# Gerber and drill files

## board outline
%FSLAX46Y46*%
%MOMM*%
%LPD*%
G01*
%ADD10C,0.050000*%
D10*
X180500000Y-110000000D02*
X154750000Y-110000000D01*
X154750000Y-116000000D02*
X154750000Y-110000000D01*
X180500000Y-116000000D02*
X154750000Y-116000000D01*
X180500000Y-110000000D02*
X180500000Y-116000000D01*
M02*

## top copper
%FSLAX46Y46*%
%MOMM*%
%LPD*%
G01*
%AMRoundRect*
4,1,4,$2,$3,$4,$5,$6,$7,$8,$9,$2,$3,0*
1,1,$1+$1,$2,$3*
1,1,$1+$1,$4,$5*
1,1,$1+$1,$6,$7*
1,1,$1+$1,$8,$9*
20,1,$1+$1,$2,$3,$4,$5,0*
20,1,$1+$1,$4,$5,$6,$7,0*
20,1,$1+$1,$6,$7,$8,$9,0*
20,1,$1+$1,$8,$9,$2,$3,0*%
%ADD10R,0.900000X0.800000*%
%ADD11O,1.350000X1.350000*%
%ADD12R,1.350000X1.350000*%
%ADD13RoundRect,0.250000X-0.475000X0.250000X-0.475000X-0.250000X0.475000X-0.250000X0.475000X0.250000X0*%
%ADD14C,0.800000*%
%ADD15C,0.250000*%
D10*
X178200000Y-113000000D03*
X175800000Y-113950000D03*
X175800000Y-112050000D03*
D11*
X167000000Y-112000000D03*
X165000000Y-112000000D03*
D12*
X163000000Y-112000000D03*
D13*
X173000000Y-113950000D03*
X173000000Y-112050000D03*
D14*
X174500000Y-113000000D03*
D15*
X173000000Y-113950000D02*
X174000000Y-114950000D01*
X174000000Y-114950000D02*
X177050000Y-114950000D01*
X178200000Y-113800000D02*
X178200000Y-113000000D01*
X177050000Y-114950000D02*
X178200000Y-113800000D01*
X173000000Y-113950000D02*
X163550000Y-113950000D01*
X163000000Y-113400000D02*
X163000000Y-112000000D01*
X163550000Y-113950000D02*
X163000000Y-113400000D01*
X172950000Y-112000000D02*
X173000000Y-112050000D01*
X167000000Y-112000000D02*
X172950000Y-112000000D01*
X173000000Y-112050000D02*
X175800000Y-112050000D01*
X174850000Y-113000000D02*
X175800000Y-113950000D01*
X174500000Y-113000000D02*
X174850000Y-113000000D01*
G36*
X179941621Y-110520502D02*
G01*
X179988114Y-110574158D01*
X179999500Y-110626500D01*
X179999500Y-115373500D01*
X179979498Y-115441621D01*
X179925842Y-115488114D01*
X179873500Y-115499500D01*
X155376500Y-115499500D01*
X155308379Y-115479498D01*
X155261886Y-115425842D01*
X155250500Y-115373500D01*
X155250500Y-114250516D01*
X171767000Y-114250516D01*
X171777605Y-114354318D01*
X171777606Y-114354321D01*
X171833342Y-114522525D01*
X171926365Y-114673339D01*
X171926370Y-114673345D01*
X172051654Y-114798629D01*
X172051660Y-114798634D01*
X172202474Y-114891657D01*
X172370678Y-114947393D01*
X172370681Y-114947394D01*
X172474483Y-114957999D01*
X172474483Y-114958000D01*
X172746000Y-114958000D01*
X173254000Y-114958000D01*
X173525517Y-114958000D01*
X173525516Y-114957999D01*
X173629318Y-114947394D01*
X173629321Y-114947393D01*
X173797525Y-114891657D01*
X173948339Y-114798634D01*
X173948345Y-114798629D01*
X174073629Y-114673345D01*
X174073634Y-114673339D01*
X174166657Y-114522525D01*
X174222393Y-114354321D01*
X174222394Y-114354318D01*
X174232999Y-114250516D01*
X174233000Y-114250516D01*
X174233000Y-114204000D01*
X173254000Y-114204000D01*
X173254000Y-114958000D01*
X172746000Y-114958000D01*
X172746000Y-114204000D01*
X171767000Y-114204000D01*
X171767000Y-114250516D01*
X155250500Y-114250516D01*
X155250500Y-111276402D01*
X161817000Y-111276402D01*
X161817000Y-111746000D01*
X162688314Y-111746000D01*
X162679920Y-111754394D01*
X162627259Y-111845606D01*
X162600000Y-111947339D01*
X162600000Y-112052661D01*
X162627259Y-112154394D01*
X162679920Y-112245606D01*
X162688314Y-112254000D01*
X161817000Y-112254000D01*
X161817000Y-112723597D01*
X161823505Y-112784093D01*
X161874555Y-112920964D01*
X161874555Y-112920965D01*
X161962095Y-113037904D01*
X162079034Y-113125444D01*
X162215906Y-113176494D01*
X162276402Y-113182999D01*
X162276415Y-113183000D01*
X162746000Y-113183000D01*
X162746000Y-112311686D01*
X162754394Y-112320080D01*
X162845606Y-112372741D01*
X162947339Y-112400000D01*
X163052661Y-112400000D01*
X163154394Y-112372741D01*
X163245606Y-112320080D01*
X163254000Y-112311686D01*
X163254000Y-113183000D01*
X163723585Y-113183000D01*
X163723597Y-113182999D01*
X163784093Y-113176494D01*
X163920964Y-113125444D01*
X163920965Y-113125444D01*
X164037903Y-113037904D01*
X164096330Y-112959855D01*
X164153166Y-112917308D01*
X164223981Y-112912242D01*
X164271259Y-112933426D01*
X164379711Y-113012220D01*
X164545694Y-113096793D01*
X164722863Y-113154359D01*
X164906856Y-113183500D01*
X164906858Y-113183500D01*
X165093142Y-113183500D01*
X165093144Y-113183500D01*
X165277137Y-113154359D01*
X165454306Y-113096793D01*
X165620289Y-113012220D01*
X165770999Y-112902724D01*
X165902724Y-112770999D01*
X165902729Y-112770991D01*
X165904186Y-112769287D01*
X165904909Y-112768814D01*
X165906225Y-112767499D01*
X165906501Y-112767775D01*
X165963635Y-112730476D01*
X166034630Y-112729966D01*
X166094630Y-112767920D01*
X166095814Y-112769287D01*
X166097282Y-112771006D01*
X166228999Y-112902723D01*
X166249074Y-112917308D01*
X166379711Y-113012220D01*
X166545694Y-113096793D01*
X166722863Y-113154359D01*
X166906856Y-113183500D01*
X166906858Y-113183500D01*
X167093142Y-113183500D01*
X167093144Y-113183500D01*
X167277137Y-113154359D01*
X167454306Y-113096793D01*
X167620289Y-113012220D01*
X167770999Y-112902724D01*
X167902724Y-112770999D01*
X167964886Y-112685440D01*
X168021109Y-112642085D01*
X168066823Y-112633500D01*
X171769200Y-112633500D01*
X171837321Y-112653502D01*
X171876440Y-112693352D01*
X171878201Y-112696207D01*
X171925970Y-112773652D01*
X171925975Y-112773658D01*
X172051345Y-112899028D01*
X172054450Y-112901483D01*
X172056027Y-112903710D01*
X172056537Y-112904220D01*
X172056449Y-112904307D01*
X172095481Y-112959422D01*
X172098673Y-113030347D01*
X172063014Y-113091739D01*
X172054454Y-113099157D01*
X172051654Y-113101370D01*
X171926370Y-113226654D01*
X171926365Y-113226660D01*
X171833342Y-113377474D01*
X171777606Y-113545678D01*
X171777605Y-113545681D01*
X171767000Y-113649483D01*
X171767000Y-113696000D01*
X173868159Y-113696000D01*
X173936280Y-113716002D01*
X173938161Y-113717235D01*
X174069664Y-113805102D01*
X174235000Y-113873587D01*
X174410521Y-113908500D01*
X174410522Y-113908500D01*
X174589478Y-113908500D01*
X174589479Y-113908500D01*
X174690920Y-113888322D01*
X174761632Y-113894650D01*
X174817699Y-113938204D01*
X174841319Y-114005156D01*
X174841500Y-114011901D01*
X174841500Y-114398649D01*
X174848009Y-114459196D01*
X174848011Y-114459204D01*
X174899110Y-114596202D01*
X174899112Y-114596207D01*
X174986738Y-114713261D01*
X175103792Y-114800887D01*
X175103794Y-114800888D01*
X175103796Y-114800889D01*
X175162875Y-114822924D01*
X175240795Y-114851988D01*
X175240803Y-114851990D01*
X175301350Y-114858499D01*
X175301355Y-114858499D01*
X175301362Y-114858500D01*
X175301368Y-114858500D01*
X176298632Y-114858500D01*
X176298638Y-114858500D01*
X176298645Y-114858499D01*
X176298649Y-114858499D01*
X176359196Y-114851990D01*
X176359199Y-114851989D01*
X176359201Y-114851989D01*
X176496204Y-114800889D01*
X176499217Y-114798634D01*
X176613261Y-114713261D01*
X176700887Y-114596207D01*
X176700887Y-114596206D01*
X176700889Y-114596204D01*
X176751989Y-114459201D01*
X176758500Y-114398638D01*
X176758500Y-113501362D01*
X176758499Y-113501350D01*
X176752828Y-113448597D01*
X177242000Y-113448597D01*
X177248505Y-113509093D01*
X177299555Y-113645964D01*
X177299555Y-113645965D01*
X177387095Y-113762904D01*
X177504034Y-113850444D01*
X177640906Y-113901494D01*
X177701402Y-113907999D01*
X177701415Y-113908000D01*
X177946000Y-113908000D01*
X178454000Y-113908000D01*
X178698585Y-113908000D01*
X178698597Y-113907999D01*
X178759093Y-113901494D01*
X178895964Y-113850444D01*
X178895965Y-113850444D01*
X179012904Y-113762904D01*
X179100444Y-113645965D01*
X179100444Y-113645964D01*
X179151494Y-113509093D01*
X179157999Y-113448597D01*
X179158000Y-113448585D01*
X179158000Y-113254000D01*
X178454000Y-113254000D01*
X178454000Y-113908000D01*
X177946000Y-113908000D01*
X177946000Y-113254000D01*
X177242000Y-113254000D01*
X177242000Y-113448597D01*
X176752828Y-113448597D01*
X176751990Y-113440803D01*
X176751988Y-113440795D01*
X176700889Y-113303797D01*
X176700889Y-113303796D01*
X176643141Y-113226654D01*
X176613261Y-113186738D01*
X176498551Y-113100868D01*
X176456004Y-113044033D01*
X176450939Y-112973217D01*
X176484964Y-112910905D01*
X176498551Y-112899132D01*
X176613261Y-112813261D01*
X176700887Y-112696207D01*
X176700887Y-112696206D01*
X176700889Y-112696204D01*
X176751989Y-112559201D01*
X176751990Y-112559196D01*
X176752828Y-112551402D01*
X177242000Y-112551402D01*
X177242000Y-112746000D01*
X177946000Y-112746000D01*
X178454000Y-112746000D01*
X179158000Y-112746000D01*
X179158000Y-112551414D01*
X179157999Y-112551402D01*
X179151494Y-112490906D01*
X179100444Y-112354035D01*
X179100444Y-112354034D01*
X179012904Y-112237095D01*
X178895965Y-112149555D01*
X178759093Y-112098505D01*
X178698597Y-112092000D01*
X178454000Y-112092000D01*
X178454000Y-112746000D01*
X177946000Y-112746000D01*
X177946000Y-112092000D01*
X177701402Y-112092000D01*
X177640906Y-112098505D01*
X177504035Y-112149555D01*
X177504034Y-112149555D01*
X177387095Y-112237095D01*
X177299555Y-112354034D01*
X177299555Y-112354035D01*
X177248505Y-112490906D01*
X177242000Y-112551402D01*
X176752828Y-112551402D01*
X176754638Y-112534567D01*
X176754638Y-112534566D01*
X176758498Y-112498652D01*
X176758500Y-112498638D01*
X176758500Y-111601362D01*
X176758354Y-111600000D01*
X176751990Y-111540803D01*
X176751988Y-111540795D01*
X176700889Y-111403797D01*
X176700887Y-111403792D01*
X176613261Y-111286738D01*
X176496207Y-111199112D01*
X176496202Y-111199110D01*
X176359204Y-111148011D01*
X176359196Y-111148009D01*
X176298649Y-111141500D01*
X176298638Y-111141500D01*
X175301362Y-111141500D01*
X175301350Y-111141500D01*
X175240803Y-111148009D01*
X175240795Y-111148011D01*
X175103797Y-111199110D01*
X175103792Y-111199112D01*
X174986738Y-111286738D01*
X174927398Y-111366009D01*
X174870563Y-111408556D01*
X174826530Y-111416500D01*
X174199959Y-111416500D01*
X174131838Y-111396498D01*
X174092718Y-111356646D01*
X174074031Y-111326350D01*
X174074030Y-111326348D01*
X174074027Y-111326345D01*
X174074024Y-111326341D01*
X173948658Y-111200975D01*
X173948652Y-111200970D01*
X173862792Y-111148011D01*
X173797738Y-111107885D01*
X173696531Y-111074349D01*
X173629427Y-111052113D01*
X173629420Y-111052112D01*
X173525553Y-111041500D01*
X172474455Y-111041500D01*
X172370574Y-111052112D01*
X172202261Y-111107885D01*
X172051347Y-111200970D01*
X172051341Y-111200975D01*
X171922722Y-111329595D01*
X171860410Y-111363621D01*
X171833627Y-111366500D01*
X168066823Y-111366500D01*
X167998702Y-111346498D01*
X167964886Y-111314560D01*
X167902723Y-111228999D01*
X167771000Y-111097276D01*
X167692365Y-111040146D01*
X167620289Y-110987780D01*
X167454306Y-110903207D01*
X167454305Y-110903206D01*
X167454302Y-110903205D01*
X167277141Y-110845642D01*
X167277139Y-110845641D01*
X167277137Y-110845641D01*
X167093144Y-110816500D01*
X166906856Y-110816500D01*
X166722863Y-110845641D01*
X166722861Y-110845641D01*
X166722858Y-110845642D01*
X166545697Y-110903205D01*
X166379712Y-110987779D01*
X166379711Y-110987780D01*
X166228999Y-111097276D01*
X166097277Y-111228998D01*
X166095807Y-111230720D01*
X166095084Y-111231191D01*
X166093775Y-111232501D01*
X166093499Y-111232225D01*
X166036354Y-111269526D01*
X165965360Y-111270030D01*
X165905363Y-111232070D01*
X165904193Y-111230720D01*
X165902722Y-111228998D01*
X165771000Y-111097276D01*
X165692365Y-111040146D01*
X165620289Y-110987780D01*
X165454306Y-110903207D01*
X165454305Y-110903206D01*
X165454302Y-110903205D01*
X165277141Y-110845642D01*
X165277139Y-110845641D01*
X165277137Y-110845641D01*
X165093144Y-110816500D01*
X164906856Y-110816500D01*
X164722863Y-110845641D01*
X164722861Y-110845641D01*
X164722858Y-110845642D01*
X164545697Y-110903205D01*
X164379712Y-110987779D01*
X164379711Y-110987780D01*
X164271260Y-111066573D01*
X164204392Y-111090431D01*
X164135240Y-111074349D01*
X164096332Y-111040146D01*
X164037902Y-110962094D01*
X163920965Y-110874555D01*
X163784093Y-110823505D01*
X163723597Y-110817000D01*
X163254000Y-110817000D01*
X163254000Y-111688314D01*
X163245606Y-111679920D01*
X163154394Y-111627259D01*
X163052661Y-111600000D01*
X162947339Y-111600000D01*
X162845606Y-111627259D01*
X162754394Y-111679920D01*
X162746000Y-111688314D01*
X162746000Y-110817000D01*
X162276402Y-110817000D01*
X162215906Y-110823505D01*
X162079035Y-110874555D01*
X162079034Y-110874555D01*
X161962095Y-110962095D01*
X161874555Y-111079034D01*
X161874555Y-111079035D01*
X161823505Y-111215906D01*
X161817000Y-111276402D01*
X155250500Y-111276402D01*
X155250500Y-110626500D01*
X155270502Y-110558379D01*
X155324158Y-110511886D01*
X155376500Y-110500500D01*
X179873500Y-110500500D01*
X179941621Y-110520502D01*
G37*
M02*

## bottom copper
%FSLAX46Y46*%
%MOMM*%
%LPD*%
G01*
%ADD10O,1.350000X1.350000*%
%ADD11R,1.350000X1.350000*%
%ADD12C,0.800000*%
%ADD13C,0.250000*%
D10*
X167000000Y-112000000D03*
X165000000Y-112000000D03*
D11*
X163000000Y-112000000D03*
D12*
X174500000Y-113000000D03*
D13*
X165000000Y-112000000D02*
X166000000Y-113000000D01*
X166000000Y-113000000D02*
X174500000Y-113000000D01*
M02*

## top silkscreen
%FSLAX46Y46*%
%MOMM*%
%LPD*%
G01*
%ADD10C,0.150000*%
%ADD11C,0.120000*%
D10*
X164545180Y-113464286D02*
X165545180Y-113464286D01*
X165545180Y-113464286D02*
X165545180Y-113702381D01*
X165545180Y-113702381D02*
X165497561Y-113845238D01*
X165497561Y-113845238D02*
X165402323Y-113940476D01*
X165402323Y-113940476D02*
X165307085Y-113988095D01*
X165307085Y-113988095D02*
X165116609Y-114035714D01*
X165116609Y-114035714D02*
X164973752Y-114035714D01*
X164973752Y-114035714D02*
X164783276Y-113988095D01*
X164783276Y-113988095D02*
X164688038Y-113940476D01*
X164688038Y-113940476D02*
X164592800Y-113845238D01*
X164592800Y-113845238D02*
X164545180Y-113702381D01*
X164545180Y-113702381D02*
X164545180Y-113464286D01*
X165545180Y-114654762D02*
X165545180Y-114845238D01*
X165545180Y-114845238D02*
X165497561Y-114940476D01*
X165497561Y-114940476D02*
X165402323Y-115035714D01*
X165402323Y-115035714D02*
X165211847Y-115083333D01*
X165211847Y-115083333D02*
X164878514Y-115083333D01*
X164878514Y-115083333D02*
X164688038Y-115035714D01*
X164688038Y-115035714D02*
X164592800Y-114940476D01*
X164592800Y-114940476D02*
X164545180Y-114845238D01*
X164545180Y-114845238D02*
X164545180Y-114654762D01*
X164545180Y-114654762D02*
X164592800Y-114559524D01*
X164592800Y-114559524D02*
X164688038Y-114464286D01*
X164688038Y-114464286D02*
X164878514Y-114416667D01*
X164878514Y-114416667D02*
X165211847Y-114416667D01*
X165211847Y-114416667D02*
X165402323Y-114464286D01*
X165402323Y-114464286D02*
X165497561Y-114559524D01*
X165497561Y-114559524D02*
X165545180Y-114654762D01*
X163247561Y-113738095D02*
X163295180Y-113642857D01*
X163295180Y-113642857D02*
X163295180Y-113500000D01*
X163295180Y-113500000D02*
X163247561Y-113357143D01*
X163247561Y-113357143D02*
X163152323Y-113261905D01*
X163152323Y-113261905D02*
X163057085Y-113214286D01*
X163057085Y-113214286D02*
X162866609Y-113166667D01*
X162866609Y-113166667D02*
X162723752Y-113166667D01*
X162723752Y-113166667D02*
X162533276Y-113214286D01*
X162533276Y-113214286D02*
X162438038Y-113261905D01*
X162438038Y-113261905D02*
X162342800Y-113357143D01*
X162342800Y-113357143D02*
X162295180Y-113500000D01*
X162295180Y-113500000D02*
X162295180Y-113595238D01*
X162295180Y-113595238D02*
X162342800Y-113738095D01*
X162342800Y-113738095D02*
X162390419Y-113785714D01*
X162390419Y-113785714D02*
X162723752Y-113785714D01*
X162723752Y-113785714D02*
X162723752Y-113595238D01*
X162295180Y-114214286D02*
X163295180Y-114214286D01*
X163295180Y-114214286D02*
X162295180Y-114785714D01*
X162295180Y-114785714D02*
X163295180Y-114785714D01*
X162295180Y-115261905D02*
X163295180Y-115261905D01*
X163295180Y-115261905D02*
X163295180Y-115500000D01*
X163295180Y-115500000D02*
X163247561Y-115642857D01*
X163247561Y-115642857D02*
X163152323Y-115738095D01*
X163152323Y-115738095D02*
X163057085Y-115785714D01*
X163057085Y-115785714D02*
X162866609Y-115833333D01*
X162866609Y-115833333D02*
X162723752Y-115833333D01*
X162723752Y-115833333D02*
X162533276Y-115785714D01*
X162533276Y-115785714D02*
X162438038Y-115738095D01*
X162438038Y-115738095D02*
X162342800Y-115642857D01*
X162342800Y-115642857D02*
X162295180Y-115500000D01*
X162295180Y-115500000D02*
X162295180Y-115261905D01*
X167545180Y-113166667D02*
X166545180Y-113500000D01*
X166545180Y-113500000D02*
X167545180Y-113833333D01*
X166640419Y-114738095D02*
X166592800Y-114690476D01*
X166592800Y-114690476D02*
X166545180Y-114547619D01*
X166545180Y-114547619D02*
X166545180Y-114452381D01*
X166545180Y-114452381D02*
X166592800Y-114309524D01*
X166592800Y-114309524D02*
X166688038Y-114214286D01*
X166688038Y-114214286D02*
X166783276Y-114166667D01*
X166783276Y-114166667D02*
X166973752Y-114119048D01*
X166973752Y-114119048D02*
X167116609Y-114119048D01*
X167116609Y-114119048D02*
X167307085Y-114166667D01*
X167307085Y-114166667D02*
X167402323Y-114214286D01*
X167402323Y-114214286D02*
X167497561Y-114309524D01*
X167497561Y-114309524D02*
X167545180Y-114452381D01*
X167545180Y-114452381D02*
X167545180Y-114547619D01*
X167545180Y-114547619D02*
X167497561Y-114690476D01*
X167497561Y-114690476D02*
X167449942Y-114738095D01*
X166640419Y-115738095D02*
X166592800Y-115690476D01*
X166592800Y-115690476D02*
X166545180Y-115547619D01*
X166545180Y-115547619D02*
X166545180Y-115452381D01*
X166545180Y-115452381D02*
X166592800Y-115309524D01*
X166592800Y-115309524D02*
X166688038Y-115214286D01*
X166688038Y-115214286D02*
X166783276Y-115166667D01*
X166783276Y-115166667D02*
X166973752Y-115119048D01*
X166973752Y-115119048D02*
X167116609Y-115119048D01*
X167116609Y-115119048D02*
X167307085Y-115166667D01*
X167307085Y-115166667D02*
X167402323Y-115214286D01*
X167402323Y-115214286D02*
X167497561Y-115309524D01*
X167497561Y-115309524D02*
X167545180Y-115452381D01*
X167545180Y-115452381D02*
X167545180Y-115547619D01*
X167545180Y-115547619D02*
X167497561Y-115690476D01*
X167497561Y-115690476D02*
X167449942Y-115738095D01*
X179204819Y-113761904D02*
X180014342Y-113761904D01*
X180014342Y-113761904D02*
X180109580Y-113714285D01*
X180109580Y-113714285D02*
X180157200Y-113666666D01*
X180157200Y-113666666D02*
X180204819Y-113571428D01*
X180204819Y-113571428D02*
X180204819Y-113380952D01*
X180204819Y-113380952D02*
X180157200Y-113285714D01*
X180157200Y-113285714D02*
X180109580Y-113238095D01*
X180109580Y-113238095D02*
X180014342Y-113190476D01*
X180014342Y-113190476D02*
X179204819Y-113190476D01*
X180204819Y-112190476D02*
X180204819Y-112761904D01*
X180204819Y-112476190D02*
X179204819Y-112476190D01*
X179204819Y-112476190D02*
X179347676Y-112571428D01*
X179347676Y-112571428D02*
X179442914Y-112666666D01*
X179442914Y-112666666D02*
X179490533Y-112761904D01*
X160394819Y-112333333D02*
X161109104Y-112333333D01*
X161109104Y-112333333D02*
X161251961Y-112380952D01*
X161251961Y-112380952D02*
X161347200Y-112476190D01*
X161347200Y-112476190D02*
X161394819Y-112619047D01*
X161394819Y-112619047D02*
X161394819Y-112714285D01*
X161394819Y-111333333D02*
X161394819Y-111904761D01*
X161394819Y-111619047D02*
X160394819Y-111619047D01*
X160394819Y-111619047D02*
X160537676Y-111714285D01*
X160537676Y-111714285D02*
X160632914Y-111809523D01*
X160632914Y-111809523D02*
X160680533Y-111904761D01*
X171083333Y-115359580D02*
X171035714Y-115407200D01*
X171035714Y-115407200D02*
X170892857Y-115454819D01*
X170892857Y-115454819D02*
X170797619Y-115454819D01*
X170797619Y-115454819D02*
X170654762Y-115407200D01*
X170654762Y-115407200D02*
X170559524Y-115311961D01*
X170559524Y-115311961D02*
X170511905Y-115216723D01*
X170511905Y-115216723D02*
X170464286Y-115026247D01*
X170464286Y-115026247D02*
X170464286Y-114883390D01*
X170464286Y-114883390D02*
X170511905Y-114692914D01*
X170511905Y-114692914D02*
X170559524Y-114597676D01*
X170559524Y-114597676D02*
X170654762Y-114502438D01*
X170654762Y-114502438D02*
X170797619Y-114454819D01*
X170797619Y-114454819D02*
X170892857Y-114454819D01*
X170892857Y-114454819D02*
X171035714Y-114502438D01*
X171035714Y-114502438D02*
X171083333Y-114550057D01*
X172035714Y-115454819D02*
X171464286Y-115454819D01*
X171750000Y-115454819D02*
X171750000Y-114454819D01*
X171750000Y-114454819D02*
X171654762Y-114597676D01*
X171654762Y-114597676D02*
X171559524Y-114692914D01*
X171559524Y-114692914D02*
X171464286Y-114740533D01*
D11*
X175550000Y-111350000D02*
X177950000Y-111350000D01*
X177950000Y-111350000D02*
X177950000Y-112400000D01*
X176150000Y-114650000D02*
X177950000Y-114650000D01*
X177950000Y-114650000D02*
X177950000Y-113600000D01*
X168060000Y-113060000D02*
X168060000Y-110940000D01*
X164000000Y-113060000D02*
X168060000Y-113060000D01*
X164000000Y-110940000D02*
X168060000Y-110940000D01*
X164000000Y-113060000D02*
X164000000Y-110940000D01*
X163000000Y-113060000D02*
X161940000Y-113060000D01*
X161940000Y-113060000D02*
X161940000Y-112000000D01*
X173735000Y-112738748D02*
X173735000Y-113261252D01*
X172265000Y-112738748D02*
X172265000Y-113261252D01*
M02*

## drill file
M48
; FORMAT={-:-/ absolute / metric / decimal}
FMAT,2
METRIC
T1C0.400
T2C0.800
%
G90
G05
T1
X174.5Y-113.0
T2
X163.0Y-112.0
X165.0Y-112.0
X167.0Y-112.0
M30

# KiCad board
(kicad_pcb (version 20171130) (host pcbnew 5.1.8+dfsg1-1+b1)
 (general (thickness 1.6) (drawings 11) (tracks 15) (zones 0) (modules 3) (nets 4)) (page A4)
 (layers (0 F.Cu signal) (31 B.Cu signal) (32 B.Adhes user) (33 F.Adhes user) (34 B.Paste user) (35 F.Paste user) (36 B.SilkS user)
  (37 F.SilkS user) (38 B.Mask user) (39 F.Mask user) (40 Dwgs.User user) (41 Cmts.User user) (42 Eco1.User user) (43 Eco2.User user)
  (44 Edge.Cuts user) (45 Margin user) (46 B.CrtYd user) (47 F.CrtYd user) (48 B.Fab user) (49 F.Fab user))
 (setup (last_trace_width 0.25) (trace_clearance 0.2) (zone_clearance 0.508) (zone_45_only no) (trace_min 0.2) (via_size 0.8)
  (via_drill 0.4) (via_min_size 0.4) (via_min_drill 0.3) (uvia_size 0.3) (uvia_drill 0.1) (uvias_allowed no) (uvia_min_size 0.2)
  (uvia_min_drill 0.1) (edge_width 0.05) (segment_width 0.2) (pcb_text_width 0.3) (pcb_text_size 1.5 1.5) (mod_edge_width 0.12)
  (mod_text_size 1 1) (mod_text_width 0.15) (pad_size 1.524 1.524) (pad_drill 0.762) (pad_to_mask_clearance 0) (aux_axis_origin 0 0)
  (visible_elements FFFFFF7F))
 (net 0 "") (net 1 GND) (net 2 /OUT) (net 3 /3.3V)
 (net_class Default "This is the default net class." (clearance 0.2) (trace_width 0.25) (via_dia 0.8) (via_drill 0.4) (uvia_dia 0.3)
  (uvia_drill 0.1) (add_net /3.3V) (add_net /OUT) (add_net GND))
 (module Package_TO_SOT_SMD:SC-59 (layer F.Cu) (at 177 113)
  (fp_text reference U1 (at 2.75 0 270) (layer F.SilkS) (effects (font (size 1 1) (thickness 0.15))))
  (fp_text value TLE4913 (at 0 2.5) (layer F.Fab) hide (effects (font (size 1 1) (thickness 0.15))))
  (fp_line (start -1.45 -1.65) (end 0.95 -1.65) (layer F.SilkS) (width 0.12))
  (fp_line (start 0.95 -1.65) (end 0.95 -0.6) (layer F.SilkS) (width 0.12))
  (fp_line (start -0.85 1.65) (end 0.95 1.65) (layer F.SilkS) (width 0.12))
  (fp_line (start 0.95 1.65) (end 0.95 0.6) (layer F.SilkS) (width 0.12))
  (pad 3 smd rect (at 1.2 0) (size 0.9 0.8) (layers F.Cu F.Paste F.Mask) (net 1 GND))
  (pad 2 smd rect (at -1.2 0.95) (size 0.9 0.8) (layers F.Cu F.Paste F.Mask) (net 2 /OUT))
  (pad 1 smd rect (at -1.2 -0.95) (size 0.9 0.8) (layers F.Cu F.Paste F.Mask) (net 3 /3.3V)))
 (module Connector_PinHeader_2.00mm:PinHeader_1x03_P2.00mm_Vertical (layer F.Cu) (at 163 112 90)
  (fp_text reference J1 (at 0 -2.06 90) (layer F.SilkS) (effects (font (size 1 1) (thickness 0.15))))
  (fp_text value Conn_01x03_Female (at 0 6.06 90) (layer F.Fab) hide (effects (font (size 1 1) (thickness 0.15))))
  (fp_line (start -1.06 5.06) (end 1.06 5.06) (layer F.SilkS) (width 0.12))
  (fp_line (start -1.06 1) (end -1.06 5.06) (layer F.SilkS) (width 0.12))
  (fp_line (start 1.06 1) (end 1.06 5.06) (layer F.SilkS) (width 0.12))
  (fp_line (start -1.06 1) (end 1.06 1) (layer F.SilkS) (width 0.12))
  (fp_line (start -1.06 0) (end -1.06 -1.06) (layer F.SilkS) (width 0.12))
  (fp_line (start -1.06 -1.06) (end 0 -1.06) (layer F.SilkS) (width 0.12))
  (pad 3 thru_hole oval (at 0 4 90) (size 1.35 1.35) (drill 0.8) (layers *.Cu *.Mask) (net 3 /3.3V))
  (pad 2 thru_hole oval (at 0 2 90) (size 1.35 1.35) (drill 0.8) (layers *.Cu *.Mask) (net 2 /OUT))
  (pad 1 thru_hole rect (at 0 0 90) (size 1.35 1.35) (drill 0.8) (layers *.Cu *.Mask) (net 1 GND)))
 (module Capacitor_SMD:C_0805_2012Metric (layer F.Cu) (at 173 113 270)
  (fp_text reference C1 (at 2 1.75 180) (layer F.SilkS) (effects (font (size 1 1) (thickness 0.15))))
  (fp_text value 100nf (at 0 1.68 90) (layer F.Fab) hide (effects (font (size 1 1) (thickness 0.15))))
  (fp_line (start -0.261252 -0.735) (end 0.261252 -0.735) (layer F.SilkS) (width 0.12))
  (fp_line (start -0.261252 0.735) (end 0.261252 0.735) (layer F.SilkS) (width 0.12))
  (pad 2 smd roundrect (at 0.95 0 270) (size 1 1.45) (layers F.Cu F.Paste F.Mask) (roundrect_rratio 0.25) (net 1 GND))
  (pad 1 smd roundrect (at -0.95 0 270) (size 1 1.45) (layers F.Cu F.Paste F.Mask) (roundrect_rratio 0.25) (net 3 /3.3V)))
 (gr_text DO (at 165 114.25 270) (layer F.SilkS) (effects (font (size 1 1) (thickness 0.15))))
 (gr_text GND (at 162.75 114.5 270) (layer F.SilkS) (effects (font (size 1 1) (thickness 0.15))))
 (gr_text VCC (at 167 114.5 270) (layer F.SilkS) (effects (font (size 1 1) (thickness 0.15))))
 (gr_line (start 180.5 110) (end 154.75 110) (layer Edge.Cuts) (width 0.05))
 (gr_line (start 154.75 116) (end 154.75 110) (layer Edge.Cuts) (width 0.05))
 (gr_line (start 180.5 116) (end 154.75 116) (layer Edge.Cuts) (width 0.05))
 (gr_line (start 180.5 110) (end 180.5 116) (layer Edge.Cuts) (width 0.05))
 (segment (start 173 113.95) (end 174 114.95) (width 0.25) (layer F.Cu) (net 1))
 (segment (start 174 114.95) (end 177.05 114.95) (width 0.25) (layer F.Cu) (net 1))
 (segment (start 178.2 113.8) (end 178.2 113) (width 0.25) (layer F.Cu) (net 1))
 (segment (start 177.05 114.95) (end 178.2 113.8) (width 0.25) (layer F.Cu) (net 1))
 (segment (start 173 113.95) (end 163.55 113.95) (width 0.25) (layer F.Cu) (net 1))
 (segment (start 163 113.4) (end 163 112) (width 0.25) (layer F.Cu) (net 1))
 (segment (start 163.55 113.95) (end 163 113.4) (width 0.25) (layer F.Cu) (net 1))
 (segment (start 172.95 112) (end 173 112.05) (width 0.25) (layer F.Cu) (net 3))
 (segment (start 167 112) (end 172.95 112) (width 0.25) (layer F.Cu) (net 3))
 (segment (start 173 112.05) (end 175.8 112.05) (width 0.25) (layer F.Cu) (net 3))
 (segment (start 165 112) (end 166 113) (width 0.25) (layer B.Cu) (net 2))
 (segment (start 166 113) (end 174.5 113) (width 0.25) (layer B.Cu) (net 2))
 (via (at 174.5 113) (size 0.8) (drill 0.4) (layers F.Cu B.Cu) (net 2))
 (segment (start 174.85 113) (end 175.8 113.95) (width 0.25) (layer F.Cu) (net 2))
 (segment (start 174.5 113) (end 174.85 113) (width 0.25) (layer F.Cu) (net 2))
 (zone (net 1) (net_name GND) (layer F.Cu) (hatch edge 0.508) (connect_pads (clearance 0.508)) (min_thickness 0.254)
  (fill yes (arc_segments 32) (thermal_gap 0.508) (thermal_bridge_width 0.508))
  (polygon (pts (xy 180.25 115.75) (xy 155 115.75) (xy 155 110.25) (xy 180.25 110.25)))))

